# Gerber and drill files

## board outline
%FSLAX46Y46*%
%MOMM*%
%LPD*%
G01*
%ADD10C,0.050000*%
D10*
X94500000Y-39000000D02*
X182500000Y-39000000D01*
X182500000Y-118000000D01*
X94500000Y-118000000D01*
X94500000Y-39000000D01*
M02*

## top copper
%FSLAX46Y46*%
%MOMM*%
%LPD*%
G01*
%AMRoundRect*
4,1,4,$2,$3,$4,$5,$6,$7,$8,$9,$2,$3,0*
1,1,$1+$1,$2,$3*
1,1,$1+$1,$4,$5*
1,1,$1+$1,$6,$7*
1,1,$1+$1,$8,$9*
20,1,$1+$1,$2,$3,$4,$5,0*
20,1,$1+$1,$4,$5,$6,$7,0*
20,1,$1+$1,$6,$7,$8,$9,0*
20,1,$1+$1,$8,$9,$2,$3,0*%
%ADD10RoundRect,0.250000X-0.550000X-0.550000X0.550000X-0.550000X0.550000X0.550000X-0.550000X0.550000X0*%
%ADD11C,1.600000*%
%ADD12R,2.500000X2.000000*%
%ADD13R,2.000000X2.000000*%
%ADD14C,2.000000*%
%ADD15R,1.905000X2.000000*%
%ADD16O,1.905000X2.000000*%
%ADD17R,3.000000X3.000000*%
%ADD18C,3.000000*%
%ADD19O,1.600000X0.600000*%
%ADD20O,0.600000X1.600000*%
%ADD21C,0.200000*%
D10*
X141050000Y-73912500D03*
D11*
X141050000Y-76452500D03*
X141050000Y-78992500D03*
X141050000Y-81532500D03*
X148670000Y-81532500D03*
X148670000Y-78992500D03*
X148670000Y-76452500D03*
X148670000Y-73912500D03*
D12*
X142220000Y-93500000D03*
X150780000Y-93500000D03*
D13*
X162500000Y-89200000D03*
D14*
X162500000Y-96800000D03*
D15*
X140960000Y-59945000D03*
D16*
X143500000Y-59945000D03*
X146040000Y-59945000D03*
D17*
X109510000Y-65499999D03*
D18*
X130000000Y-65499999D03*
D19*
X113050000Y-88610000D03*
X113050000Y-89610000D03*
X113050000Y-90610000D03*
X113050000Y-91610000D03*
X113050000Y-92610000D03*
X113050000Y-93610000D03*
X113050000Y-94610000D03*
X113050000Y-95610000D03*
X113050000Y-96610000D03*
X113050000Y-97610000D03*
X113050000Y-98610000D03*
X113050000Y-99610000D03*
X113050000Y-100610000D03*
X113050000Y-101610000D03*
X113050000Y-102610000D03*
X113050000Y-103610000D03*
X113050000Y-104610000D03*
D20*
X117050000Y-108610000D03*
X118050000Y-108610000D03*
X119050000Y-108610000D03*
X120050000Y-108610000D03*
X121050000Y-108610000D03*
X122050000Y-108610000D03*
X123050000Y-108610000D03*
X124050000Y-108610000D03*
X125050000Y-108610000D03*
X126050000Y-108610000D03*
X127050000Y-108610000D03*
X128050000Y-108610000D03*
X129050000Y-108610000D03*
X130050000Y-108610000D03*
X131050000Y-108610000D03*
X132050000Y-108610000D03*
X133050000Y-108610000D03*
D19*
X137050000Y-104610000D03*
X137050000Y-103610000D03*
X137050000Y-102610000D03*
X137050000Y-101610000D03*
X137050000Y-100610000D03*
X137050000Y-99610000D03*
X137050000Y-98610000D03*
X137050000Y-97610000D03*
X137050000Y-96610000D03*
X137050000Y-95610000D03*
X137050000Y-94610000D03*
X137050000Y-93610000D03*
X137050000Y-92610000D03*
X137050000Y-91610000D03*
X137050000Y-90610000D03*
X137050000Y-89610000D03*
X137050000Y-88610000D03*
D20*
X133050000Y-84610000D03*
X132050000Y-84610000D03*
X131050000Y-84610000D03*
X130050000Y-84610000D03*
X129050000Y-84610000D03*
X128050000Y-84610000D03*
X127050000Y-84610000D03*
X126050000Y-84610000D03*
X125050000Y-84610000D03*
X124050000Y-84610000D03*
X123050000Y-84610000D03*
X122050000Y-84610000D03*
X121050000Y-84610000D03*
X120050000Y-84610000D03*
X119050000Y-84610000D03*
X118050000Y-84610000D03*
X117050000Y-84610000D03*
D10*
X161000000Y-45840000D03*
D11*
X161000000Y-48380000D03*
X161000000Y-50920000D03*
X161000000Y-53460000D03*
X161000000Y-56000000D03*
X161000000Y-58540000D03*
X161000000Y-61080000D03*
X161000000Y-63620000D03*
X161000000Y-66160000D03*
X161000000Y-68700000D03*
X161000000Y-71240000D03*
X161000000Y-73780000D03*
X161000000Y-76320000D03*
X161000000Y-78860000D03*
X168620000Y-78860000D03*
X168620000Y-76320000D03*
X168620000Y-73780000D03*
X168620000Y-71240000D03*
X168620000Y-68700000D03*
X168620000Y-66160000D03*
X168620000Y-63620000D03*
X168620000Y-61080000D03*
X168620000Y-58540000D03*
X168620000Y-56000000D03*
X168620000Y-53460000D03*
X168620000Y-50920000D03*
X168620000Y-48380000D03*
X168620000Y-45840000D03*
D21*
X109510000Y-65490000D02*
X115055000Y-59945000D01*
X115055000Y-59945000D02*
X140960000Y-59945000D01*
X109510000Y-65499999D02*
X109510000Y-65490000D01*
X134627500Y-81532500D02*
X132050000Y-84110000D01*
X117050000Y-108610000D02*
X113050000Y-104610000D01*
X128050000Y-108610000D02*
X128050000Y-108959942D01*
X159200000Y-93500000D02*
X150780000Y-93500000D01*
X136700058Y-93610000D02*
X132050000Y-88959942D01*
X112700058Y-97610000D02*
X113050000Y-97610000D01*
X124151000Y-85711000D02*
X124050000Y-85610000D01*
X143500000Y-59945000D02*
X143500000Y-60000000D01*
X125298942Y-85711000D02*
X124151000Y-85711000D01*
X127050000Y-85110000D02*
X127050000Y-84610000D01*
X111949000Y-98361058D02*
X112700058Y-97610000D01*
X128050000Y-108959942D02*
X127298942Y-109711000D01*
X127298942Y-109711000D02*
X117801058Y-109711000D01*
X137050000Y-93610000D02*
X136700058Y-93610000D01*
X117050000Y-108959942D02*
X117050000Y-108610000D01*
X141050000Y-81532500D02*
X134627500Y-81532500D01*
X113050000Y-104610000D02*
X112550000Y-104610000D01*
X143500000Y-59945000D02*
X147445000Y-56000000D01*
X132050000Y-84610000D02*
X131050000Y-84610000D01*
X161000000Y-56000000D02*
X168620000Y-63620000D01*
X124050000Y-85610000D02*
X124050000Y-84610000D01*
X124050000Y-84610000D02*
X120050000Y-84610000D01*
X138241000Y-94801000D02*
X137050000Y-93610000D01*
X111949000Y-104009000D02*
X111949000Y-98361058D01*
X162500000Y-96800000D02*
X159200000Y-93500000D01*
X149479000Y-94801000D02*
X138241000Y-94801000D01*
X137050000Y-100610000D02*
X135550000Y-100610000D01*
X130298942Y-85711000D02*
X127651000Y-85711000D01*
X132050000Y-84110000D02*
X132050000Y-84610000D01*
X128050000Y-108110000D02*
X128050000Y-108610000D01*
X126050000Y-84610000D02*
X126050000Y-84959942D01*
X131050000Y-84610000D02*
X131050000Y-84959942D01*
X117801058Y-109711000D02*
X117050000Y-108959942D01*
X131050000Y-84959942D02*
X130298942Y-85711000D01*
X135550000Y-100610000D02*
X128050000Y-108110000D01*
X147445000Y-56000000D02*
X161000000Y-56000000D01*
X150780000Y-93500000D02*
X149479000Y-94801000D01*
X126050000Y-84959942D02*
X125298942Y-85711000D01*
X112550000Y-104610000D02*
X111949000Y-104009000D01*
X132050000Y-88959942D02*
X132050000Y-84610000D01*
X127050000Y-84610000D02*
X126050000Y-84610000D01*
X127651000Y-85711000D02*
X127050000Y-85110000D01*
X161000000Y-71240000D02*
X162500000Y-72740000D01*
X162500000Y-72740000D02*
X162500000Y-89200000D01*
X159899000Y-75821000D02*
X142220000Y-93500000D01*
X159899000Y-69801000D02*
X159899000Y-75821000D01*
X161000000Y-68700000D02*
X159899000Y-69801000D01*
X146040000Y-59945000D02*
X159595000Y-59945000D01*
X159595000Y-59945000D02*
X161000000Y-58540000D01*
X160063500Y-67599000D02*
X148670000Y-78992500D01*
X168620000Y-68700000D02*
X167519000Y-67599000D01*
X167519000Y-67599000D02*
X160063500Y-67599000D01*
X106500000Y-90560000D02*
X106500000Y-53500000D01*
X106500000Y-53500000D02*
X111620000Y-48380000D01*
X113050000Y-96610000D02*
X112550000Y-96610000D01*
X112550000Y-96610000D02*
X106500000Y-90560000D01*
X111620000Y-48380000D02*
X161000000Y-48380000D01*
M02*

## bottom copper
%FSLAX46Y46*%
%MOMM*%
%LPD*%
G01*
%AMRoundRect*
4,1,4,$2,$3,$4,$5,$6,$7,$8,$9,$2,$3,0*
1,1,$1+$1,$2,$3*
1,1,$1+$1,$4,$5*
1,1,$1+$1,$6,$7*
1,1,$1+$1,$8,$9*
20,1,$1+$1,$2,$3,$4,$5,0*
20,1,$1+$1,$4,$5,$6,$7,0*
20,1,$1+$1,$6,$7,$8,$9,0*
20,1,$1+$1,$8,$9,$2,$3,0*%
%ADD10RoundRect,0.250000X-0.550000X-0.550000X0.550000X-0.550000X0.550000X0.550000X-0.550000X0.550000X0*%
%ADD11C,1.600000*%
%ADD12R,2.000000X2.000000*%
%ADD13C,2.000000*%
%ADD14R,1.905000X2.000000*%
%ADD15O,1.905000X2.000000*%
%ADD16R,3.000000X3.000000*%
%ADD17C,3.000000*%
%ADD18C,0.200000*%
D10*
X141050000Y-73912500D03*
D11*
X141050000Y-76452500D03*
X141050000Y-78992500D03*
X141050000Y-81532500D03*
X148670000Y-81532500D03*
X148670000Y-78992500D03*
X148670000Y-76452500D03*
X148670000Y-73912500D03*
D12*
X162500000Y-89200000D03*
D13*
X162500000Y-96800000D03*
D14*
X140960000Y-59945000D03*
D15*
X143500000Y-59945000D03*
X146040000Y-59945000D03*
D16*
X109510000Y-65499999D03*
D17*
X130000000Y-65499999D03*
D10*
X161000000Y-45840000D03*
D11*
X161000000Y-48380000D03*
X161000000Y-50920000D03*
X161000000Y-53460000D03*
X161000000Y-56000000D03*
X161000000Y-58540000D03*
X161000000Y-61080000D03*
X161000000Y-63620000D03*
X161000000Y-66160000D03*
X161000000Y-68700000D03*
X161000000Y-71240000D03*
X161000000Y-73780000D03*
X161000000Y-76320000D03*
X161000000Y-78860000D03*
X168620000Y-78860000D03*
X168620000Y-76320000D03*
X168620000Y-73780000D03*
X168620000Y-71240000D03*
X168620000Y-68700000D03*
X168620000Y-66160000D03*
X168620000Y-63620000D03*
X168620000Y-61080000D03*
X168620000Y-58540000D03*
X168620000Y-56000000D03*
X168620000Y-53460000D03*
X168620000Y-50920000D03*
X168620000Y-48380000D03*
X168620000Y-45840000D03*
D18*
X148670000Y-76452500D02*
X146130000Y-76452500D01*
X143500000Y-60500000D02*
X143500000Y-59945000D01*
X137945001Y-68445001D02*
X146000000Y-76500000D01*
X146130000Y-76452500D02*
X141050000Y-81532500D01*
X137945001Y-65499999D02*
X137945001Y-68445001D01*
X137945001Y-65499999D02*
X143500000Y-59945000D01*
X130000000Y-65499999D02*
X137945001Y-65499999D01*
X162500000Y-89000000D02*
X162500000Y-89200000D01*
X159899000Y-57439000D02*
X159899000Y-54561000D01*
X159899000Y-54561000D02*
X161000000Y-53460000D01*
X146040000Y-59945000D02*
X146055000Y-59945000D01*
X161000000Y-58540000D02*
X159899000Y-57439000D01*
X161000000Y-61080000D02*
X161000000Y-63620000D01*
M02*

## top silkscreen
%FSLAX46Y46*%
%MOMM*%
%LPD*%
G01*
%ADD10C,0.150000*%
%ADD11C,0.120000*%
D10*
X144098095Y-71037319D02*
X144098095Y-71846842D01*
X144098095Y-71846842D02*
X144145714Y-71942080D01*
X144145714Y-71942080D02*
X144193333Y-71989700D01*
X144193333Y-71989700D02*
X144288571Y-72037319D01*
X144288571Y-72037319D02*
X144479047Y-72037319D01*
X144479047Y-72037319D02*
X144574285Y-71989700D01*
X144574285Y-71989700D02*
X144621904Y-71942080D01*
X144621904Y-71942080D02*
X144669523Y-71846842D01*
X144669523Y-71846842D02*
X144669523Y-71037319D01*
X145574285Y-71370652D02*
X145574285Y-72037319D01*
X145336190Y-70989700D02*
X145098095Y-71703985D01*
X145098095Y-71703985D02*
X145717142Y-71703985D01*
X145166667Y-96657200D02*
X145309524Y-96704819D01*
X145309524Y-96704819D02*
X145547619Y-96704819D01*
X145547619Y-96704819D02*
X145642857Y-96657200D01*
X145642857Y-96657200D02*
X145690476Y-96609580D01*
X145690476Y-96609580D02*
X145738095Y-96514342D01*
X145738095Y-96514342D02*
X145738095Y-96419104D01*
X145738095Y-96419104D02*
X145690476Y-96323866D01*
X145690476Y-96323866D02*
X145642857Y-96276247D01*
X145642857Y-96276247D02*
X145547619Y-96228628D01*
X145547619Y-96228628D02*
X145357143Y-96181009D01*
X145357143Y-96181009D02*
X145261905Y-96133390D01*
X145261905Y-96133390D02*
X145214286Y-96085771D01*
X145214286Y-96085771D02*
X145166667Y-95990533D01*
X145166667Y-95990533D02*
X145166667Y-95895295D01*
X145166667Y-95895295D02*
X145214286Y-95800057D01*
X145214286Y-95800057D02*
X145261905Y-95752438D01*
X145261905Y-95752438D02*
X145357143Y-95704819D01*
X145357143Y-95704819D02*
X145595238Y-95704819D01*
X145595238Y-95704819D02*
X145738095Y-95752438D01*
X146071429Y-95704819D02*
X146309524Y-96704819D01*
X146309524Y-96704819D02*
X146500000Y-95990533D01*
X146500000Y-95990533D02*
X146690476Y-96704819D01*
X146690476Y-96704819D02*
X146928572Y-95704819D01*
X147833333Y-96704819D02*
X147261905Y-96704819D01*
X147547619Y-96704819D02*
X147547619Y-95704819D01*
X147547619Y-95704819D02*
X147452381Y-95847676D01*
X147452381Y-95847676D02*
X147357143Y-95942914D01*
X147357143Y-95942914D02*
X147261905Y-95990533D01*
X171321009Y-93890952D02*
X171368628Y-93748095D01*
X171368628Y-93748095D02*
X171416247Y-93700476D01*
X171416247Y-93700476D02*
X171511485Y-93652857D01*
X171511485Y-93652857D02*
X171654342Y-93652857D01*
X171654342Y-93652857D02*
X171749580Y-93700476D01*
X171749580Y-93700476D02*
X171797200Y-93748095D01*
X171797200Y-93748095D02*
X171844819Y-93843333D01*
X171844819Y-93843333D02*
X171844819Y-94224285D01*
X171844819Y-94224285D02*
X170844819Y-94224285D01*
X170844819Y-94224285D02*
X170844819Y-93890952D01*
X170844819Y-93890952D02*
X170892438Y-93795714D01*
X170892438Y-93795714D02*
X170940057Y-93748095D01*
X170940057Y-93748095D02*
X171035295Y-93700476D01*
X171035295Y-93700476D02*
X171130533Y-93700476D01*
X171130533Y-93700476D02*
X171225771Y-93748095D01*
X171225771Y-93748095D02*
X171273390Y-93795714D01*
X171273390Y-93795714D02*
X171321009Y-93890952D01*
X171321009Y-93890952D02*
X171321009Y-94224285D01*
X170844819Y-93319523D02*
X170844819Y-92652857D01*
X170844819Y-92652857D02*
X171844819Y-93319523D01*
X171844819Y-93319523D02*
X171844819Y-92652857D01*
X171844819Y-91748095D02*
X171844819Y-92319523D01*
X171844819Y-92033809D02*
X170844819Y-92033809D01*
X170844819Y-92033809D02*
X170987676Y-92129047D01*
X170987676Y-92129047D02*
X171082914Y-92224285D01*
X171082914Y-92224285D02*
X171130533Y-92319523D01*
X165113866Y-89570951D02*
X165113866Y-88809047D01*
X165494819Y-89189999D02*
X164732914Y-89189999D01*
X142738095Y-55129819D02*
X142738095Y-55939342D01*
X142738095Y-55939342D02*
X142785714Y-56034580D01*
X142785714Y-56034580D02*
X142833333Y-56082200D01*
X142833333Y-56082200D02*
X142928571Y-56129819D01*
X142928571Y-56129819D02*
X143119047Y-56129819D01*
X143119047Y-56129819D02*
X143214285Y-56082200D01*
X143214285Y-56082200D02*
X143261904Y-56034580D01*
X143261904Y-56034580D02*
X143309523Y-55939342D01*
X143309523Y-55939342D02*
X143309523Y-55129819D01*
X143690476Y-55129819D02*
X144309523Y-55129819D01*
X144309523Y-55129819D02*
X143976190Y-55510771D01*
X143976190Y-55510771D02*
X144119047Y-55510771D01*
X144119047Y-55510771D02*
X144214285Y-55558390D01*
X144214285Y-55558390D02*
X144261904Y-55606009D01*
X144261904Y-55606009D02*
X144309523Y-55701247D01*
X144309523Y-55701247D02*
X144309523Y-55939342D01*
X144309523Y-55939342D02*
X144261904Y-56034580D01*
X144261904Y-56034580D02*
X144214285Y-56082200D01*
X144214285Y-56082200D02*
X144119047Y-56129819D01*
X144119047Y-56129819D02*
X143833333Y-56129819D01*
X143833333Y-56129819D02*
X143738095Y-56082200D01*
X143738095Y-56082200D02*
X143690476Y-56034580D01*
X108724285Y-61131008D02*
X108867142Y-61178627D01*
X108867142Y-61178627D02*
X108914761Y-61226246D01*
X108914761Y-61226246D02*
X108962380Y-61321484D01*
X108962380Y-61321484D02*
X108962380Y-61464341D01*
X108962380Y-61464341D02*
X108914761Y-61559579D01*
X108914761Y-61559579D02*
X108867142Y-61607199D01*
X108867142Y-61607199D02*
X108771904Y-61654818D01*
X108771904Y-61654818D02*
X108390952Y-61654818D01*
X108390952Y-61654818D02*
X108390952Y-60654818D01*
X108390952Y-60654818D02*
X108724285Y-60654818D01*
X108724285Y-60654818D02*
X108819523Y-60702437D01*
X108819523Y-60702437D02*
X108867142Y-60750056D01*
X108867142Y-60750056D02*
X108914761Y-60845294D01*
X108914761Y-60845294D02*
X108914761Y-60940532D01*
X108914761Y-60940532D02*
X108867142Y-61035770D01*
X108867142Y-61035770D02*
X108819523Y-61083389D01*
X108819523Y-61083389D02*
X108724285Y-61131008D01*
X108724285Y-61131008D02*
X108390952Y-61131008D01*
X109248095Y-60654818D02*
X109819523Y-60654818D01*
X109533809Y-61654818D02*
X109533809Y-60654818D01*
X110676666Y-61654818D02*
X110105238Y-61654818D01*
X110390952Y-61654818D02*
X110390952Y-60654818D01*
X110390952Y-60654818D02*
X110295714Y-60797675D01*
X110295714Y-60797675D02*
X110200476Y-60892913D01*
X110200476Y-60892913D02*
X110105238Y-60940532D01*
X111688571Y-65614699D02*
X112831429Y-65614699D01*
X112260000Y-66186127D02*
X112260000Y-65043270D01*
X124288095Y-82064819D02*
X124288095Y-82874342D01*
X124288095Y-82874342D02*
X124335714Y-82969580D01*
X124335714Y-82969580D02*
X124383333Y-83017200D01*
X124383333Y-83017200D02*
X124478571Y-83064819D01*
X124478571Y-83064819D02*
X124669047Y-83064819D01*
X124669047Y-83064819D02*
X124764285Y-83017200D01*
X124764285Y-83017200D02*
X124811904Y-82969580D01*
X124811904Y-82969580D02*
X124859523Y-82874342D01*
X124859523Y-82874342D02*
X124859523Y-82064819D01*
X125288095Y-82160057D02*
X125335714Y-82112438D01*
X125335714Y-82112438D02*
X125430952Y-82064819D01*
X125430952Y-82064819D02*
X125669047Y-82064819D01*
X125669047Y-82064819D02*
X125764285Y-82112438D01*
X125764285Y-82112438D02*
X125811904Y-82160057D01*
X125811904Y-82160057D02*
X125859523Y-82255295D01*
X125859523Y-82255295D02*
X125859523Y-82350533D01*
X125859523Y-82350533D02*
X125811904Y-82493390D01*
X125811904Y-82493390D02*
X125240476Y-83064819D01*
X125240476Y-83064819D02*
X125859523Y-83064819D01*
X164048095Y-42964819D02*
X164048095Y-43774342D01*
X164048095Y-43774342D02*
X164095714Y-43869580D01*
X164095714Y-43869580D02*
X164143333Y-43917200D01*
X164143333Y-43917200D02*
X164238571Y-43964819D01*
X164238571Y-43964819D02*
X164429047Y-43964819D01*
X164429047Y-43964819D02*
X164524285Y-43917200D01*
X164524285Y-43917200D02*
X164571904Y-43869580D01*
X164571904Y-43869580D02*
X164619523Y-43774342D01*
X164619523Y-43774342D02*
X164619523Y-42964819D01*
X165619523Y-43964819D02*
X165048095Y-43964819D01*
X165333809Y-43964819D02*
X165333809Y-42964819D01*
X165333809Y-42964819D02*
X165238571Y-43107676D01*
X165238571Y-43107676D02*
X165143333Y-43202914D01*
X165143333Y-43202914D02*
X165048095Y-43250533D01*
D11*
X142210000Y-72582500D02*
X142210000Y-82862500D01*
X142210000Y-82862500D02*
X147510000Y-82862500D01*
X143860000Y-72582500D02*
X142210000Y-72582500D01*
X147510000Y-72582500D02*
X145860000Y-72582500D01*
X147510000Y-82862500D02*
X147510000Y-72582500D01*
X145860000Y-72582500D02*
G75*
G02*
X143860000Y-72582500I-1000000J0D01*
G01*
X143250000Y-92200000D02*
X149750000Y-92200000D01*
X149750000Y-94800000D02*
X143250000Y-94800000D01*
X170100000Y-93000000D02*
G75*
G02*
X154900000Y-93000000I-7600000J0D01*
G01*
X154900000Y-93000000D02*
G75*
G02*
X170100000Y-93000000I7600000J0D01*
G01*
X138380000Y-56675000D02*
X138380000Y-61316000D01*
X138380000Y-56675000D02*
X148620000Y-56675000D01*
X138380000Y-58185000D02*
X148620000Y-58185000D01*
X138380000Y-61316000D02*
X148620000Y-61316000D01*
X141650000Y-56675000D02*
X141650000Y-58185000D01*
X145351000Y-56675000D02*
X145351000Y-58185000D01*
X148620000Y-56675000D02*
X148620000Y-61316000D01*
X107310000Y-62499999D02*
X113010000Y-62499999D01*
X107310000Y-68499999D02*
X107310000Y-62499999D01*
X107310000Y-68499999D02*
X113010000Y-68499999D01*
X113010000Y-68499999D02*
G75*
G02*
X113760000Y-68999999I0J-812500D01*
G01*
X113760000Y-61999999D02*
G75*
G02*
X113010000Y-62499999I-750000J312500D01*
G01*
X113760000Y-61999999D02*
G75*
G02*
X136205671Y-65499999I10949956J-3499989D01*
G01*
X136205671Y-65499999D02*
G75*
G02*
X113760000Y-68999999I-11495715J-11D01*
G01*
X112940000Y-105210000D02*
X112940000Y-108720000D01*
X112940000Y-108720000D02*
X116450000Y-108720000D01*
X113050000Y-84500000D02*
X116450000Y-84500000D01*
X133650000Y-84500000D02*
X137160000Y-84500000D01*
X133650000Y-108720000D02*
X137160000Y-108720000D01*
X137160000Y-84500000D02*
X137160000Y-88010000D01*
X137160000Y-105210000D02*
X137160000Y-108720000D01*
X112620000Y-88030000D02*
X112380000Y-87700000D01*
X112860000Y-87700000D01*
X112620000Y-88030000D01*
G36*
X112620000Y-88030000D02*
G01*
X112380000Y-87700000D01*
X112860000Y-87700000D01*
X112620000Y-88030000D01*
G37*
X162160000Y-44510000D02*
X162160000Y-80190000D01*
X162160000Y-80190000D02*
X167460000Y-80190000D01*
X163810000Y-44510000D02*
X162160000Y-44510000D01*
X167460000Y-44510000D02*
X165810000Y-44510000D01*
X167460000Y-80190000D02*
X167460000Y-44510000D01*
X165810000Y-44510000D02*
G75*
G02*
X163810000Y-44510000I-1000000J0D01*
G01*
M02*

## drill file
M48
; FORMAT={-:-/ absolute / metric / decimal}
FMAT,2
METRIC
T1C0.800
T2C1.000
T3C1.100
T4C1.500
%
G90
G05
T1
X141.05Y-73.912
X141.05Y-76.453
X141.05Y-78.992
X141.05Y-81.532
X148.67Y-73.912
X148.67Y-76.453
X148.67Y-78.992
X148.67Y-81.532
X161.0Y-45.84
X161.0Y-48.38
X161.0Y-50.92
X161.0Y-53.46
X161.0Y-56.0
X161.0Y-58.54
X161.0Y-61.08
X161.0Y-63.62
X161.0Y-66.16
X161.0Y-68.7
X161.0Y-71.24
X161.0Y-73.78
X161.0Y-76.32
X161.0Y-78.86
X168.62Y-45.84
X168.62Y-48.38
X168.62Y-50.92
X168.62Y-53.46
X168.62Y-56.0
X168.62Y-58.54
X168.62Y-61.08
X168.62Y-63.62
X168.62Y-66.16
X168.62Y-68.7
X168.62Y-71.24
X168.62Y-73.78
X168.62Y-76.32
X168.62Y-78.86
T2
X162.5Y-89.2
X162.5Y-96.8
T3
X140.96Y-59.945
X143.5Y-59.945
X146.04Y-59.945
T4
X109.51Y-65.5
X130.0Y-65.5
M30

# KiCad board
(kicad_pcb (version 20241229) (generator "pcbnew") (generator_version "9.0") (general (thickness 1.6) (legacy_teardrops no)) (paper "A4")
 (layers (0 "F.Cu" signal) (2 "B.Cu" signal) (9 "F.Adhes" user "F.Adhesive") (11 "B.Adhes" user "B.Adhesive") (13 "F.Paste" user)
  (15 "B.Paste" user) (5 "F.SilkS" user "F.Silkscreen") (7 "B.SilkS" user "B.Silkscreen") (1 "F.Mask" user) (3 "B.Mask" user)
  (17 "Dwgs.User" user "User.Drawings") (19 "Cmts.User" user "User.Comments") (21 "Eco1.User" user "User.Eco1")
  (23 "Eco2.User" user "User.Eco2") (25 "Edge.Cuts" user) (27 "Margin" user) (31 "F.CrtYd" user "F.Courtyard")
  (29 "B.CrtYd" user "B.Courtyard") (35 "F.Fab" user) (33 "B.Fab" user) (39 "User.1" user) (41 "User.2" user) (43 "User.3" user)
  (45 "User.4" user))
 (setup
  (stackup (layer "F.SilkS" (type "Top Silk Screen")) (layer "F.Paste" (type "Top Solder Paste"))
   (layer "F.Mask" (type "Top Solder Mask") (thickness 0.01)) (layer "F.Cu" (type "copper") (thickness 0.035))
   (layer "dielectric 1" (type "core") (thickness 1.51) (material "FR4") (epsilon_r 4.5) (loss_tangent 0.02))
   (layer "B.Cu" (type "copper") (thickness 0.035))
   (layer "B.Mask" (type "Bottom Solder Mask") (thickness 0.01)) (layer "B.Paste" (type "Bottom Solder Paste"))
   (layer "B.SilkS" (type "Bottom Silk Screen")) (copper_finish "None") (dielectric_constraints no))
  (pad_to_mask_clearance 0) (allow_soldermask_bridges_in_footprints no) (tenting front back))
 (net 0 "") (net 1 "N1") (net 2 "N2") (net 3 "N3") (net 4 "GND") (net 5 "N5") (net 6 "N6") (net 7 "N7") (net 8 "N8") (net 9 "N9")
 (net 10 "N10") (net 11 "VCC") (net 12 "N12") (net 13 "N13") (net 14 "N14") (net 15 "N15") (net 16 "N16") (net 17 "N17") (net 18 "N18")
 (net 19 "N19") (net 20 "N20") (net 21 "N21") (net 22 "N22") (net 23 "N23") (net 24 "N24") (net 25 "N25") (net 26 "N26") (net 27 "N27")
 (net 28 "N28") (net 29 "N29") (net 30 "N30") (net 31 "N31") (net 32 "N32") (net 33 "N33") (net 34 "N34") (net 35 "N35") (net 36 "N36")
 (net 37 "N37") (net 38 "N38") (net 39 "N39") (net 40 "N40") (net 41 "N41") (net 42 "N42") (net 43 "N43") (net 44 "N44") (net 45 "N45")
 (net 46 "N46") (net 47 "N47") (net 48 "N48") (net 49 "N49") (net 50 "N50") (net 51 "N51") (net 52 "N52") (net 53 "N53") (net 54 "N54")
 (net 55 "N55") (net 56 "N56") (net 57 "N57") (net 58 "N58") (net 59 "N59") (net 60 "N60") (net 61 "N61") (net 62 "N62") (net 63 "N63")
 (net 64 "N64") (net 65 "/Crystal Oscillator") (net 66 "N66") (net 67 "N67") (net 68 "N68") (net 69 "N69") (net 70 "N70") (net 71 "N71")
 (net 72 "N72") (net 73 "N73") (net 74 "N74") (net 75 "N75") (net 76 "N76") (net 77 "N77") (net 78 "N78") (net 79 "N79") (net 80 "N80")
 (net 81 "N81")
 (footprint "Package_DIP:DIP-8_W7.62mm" (layer "F.Cu") (at 141.05 73.9125)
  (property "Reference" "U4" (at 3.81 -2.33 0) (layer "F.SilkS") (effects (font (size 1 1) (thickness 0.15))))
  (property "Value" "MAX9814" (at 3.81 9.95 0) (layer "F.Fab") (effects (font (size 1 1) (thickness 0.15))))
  (fp_line (start 1.16 -1.33) (end 1.16 8.95) (stroke (width 0.12) (type solid)) (layer "F.SilkS"))
  (fp_line (start 1.16 8.95) (end 6.46 8.95) (stroke (width 0.12) (type solid)) (layer "F.SilkS"))
  (fp_line (start 2.81 -1.33) (end 1.16 -1.33) (stroke (width 0.12) (type solid)) (layer "F.SilkS"))
  (fp_line (start 6.46 -1.33) (end 4.81 -1.33) (stroke (width 0.12) (type solid)) (layer "F.SilkS"))
  (fp_line (start 6.46 8.95) (end 6.46 -1.33) (stroke (width 0.12) (type solid)) (layer "F.SilkS"))
  (fp_arc (start 4.81 -1.33) (mid 3.81 -0.33) (end 2.81 -1.33) (stroke (width 0.12) (type solid)) (layer "F.SilkS"))
  (pad "1" thru_hole roundrect (at 0 0) (size 1.6 1.6) (drill 0.8) (layers "*.Cu" "*.Mask") (remove_unused_layers no)
   (roundrect_rratio 0.15625) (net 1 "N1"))
  (pad "2" thru_hole circle (at 0 2.54) (size 1.6 1.6) (drill 0.8) (layers "*.Cu" "*.Mask") (remove_unused_layers no) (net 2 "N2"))
  (pad "3" thru_hole circle (at 0 5.08) (size 1.6 1.6) (drill 0.8) (layers "*.Cu" "*.Mask") (remove_unused_layers no) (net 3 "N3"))
  (pad "4" thru_hole circle (at 0 7.62) (size 1.6 1.6) (drill 0.8) (layers "*.Cu" "*.Mask") (remove_unused_layers no) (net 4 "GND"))
  (pad "5" thru_hole circle (at 7.62 7.62) (size 1.6 1.6) (drill 0.8) (layers "*.Cu" "*.Mask") (remove_unused_layers no) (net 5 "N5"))
  (pad "6" thru_hole circle (at 7.62 5.08) (size 1.6 1.6) (drill 0.8) (layers "*.Cu" "*.Mask") (remove_unused_layers no) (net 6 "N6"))
  (pad "7" thru_hole circle (at 7.62 2.54) (size 1.6 1.6) (drill 0.8) (layers "*.Cu" "*.Mask") (remove_unused_layers no) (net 4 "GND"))
  (pad "8" thru_hole circle (at 7.62 0) (size 1.6 1.6) (drill 0.8) (layers "*.Cu" "*.Mask") (remove_unused_layers no) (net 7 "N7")))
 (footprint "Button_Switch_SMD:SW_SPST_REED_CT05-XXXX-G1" (layer "F.Cu") (at 146.5 93.5)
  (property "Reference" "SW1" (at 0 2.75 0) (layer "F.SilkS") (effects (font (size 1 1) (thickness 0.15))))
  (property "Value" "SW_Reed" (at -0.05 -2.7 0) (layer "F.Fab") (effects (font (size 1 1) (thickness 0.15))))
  (fp_line (start -3.25 -1.3) (end 3.25 -1.3) (stroke (width 0.12) (type solid)) (layer "F.SilkS"))
  (fp_line (start 3.25 1.3) (end -3.25 1.3) (stroke (width 0.12) (type solid)) (layer "F.SilkS"))
  (pad "1" smd rect (at -4.28 0) (size 2.5 2) (layers "F.Cu" "F.Mask" "F.Paste") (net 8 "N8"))
  (pad "2" smd rect (at 4.28 0) (size 2.5 2) (layers "F.Cu" "F.Mask" "F.Paste") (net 4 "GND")))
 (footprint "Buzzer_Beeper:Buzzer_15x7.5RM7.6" (layer "F.Cu") (at 162.5 89.2 -90)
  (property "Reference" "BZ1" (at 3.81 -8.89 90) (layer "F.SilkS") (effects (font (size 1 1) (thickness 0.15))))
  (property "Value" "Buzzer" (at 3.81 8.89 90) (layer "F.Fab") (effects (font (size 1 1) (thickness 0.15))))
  (fp_circle (center 3.8 0) (end 11.4 0) (stroke (width 0.12) (type solid)) (fill no) (layer "F.SilkS"))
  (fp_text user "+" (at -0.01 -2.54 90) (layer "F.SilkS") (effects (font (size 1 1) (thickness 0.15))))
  (pad "1" thru_hole rect (at 0 0 270) (size 2 2) (drill 1) (layers "*.Cu" "*.Mask") (remove_unused_layers no) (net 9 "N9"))
  (pad "2" thru_hole circle (at 7.6 0 270) (size 2 2) (drill 1) (layers "*.Cu" "*.Mask") (remove_unused_layers no) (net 4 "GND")))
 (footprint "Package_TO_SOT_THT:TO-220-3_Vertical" (layer "F.Cu") (at 140.96 59.945)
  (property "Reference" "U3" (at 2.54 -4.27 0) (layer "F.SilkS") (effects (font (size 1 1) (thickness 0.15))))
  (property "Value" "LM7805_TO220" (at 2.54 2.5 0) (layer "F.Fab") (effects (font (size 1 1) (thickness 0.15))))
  (fp_line (start -2.58 -3.27) (end -2.58 1.371) (stroke (width 0.12) (type solid)) (layer "F.SilkS"))
  (fp_line (start -2.58 -3.27) (end 7.66 -3.27) (stroke (width 0.12) (type solid)) (layer "F.SilkS"))
  (fp_line (start -2.58 -1.76) (end 7.66 -1.76) (stroke (width 0.12) (type solid)) (layer "F.SilkS"))
  (fp_line (start -2.58 1.371) (end 7.66 1.371) (stroke (width 0.12) (type solid)) (layer "F.SilkS"))
  (fp_line (start 0.69 -3.27) (end 0.69 -1.76) (stroke (width 0.12) (type solid)) (layer "F.SilkS"))
  (fp_line (start 4.391 -3.27) (end 4.391 -1.76) (stroke (width 0.12) (type solid)) (layer "F.SilkS"))
  (fp_line (start 7.66 -3.27) (end 7.66 1.371) (stroke (width 0.12) (type solid)) (layer "F.SilkS"))
  (pad "1" thru_hole rect (at 0 0) (size 1.905 2) (drill 1.1) (layers "*.Cu" "*.Mask") (remove_unused_layers no) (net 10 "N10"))
  (pad "2" thru_hole oval (at 2.54 0) (size 1.905 2) (drill 1.1) (layers "*.Cu" "*.Mask") (remove_unused_layers no) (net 4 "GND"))
  (pad "3" thru_hole oval (at 5.08 0) (size 1.905 2) (drill 1.1) (layers "*.Cu" "*.Mask") (remove_unused_layers no) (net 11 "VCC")))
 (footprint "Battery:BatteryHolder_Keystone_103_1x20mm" (layer "F.Cu") (at 109.51 65.499999)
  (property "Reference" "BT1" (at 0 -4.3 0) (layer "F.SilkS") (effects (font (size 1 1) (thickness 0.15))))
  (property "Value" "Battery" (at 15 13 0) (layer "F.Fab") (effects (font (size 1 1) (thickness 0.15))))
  (fp_line (start -2.2 -3) (end 3.5 -3) (stroke (width 0.12) (type solid)) (layer "F.SilkS"))
  (fp_line (start -2.2 3) (end -2.2 -3) (stroke (width 0.12) (type solid)) (layer "F.SilkS"))
  (fp_line (start -2.2 3) (end 3.5 3) (stroke (width 0.12) (type solid)) (layer "F.SilkS"))
  (fp_arc (start 3.5 3) (mid 3.950694 3.136459) (end 4.25 3.5) (stroke (width 0.12) (type solid)) (layer "F.SilkS"))
  (fp_arc (start 4.25 -3.5) (mid 3.950694 -3.136459) (end 3.5 -3) (stroke (width 0.12) (type solid)) (layer "F.SilkS"))
  (fp_arc (start 4.25 -3.5) (mid 16.971103 -11.358466) (end 26.695671 0) (stroke (width 0.12) (type solid)) (layer "F.SilkS"))
  (fp_arc (start 26.695671 0) (mid 16.971103 11.358466) (end 4.25 3.5) (stroke (width 0.12) (type solid)) (layer "F.SilkS"))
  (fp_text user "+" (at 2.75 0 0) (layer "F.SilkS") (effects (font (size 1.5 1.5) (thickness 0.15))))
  (pad "1" thru_hole rect (at 0 0) (size 3 3) (drill 1.5) (layers "*.Cu" "*.Mask") (remove_unused_layers no) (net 10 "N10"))
  (pad "2" thru_hole circle (at 20.49 0) (size 3 3) (drill 1.5) (layers "*.Cu" "*.Mask") (remove_unused_layers no) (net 4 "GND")))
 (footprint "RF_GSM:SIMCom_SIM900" (layer "F.Cu") (at 125.05 96.61)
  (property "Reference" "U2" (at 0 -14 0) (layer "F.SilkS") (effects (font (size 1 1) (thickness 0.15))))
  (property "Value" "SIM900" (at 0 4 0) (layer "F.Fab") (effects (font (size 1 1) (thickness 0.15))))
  (fp_line (start -12.11 8.6) (end -12.11 12.11) (stroke (width 0.12) (type solid)) (layer "F.SilkS"))
  (fp_line (start -12.11 12.11) (end -8.6 12.11) (stroke (width 0.12) (type solid)) (layer "F.SilkS"))
  (fp_line (start -12 -12.11) (end -8.6 -12.11) (stroke (width 0.12) (type solid)) (layer "F.SilkS"))
  (fp_line (start 8.6 -12.11) (end 12.11 -12.11) (stroke (width 0.12) (type solid)) (layer "F.SilkS"))
  (fp_line (start 8.6 12.11) (end 12.11 12.11) (stroke (width 0.12) (type solid)) (layer "F.SilkS"))
  (fp_line (start 12.11 -12.11) (end 12.11 -8.6) (stroke (width 0.12) (type solid)) (layer "F.SilkS"))
  (fp_line (start 12.11 8.6) (end 12.11 12.11) (stroke (width 0.12) (type solid)) (layer "F.SilkS"))
  (fp_poly
   (pts (xy -12.43 -8.58) (xy -12.67 -8.91) (xy -12.19 -8.91) (xy -12.43 -8.58)) (stroke (width 0.12) (type solid)) (fill yes)
   (layer "F.SilkS"))
  (pad "1" smd oval (at -12 -8) (size 1.6 0.6) (layers "F.Cu" "F.Mask" "F.Paste") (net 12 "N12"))
  (pad "2" smd oval (at -12 -7) (size 1.6 0.6) (layers "F.Cu" "F.Mask" "F.Paste") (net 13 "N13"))
  (pad "3" smd oval (at -12 -6) (size 1.6 0.6) (layers "F.Cu" "F.Mask" "F.Paste") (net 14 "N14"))
  (pad "4" smd oval (at -12 -5) (size 1.6 0.6) (layers "F.Cu" "F.Mask" "F.Paste") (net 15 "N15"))
  (pad "5" smd oval (at -12 -4) (size 1.6 0.6) (layers "F.Cu" "F.Mask" "F.Paste") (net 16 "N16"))
  (pad "6" smd oval (at -12 -3) (size 1.6 0.6) (layers "F.Cu" "F.Mask" "F.Paste") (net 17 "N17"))
  (pad "7" smd oval (at -12 -2) (size 1.6 0.6) (layers "F.Cu" "F.Mask" "F.Paste") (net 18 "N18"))
  (pad "8" smd oval (at -12 -1) (size 1.6 0.6) (layers "F.Cu" "F.Mask" "F.Paste") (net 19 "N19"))
  (pad "9" smd oval (at -12 0) (size 1.6 0.6) (layers "F.Cu" "F.Mask" "F.Paste") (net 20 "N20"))
  (pad "10" smd oval (at -12 1) (size 1.6 0.6) (layers "F.Cu" "F.Mask" "F.Paste") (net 4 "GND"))
  (pad "11" smd oval (at -12 2) (size 1.6 0.6) (layers "F.Cu" "F.Mask" "F.Paste") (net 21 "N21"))
  (pad "12" smd oval (at -12 3) (size 1.6 0.6) (layers "F.Cu" "F.Mask" "F.Paste") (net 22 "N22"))
  (pad "13" smd oval (at -12 4) (size 1.6 0.6) (layers "F.Cu" "F.Mask" "F.Paste") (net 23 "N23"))
  (pad "14" smd oval (at -12 5) (size 1.6 0.6) (layers "F.Cu" "F.Mask" "F.Paste") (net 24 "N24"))
  (pad "15" smd oval (at -12 6) (size 1.6 0.6) (layers "F.Cu" "F.Mask" "F.Paste") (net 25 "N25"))
  (pad "16" smd oval (at -12 7) (size 1.6 0.6) (layers "F.Cu" "F.Mask" "F.Paste") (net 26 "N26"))
  (pad "17" smd oval (at -12 8) (size 1.6 0.6) (layers "F.Cu" "F.Mask" "F.Paste") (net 4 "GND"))
  (pad "18" smd oval (at -8 12) (size 0.6 1.6) (layers "F.Cu" "F.Mask" "F.Paste") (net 4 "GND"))
  (pad "19" smd oval (at -7 12) (size 0.6 1.6) (layers "F.Cu" "F.Mask" "F.Paste") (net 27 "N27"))
  (pad "20" smd oval (at -6 12) (size 0.6 1.6) (layers "F.Cu" "F.Mask" "F.Paste") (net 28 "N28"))
  (pad "21" smd oval (at -5 12) (size 0.6 1.6) (layers "F.Cu" "F.Mask" "F.Paste") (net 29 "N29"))
  (pad "22" smd oval (at -4 12) (size 0.6 1.6) (layers "F.Cu" "F.Mask" "F.Paste") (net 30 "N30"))
  (pad "23" smd oval (at -3 12) (size 0.6 1.6) (layers "F.Cu" "F.Mask" "F.Paste") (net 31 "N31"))
  (pad "24" smd oval (at -2 12) (size 0.6 1.6) (layers "F.Cu" "F.Mask" "F.Paste") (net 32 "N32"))
  (pad "25" smd oval (at -1 12) (size 0.6 1.6) (layers "F.Cu" "F.Mask" "F.Paste") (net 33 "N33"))
  (pad "26" smd oval (at 0 12) (size 0.6 1.6) (layers "F.Cu" "F.Mask" "F.Paste") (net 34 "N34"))
  (pad "27" smd oval (at 1 12) (size 0.6 1.6) (layers "F.Cu" "F.Mask" "F.Paste") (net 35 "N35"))
  (pad "28" smd oval (at 2 12) (size 0.6 1.6) (layers "F.Cu" "F.Mask" "F.Paste") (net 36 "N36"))
  (pad "29" smd oval (at 3 12) (size 0.6 1.6) (layers "F.Cu" "F.Mask" "F.Paste") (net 4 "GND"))
  (pad "30" smd oval (at 4 12) (size 0.6 1.6) (layers "F.Cu" "F.Mask" "F.Paste") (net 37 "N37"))
  (pad "31" smd oval (at 5 12) (size 0.6 1.6) (layers "F.Cu" "F.Mask" "F.Paste") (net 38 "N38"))
  (pad "32" smd oval (at 6 12) (size 0.6 1.6) (layers "F.Cu" "F.Mask" "F.Paste") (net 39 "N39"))
  (pad "33" smd oval (at 7 12) (size 0.6 1.6) (layers "F.Cu" "F.Mask" "F.Paste") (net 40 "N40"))
  (pad "34" smd oval (at 8 12) (size 0.6 1.6) (layers "F.Cu" "F.Mask" "F.Paste") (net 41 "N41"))
  (pad "35" smd oval (at 12 8) (size 1.6 0.6) (layers "F.Cu" "F.Mask" "F.Paste") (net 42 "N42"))
  (pad "36" smd oval (at 12 7) (size 1.6 0.6) (layers "F.Cu" "F.Mask" "F.Paste") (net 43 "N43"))
  (pad "37" smd oval (at 12 6) (size 1.6 0.6) (layers "F.Cu" "F.Mask" "F.Paste") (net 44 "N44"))
  (pad "38" smd oval (at 12 5) (size 1.6 0.6) (layers "F.Cu" "F.Mask" "F.Paste") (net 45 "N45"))
  (pad "39" smd oval (at 12 4) (size 1.6 0.6) (layers "F.Cu" "F.Mask" "F.Paste") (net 4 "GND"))
  (pad "40" smd oval (at 12 3) (size 1.6 0.6) (layers "F.Cu" "F.Mask" "F.Paste") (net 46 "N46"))
  (pad "41" smd oval (at 12 2) (size 1.6 0.6) (layers "F.Cu" "F.Mask" "F.Paste") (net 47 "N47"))
  (pad "42" smd oval (at 12 1) (size 1.6 0.6) (layers "F.Cu" "F.Mask" "F.Paste") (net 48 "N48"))
  (pad "43" smd oval (at 12 0) (size 1.6 0.6) (layers "F.Cu" "F.Mask" "F.Paste") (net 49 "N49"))
  (pad "44" smd oval (at 12 -1) (size 1.6 0.6) (layers "F.Cu" "F.Mask" "F.Paste") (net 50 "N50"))
  (pad "45" smd oval (at 12 -2) (size 1.6 0.6) (layers "F.Cu" "F.Mask" "F.Paste") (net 4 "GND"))
  (pad "46" smd oval (at 12 -3) (size 1.6 0.6) (layers "F.Cu" "F.Mask" "F.Paste") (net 4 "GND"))
  (pad "47" smd oval (at 12 -4) (size 1.6 0.6) (layers "F.Cu" "F.Mask" "F.Paste") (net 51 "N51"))
  (pad "48" smd oval (at 12 -5) (size 1.6 0.6) (layers "F.Cu" "F.Mask" "F.Paste") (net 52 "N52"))
  (pad "49" smd oval (at 12 -6) (size 1.6 0.6) (layers "F.Cu" "F.Mask" "F.Paste") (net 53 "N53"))
  (pad "50" smd oval (at 12 -7) (size 1.6 0.6) (layers "F.Cu" "F.Mask" "F.Paste") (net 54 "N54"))
  (pad "51" smd oval (at 12 -8) (size 1.6 0.6) (layers "F.Cu" "F.Mask" "F.Paste") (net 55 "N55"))
  (pad "52" smd oval (at 8 -12) (size 0.6 1.6) (layers "F.Cu" "F.Mask" "F.Paste") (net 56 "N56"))
  (pad "53" smd oval (at 7 -12) (size 0.6 1.6) (layers "F.Cu" "F.Mask" "F.Paste") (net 4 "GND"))
  (pad "54" smd oval (at 6 -12) (size 0.6 1.6) (layers "F.Cu" "F.Mask" "F.Paste") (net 4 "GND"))
  (pad "55" smd oval (at 5 -12) (size 0.6 1.6) (layers "F.Cu" "F.Mask" "F.Paste") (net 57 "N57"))
  (pad "56" smd oval (at 4 -12) (size 0.6 1.6) (layers "F.Cu" "F.Mask" "F.Paste") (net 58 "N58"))
  (pad "57" smd oval (at 3 -12) (size 0.6 1.6) (layers "F.Cu" "F.Mask" "F.Paste") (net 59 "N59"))
  (pad "58" smd oval (at 2 -12) (size 0.6 1.6) (layers "F.Cu" "F.Mask" "F.Paste") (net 4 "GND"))
  (pad "59" smd oval (at 1 -12) (size 0.6 1.6) (layers "F.Cu" "F.Mask" "F.Paste") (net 4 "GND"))
  (pad "60" smd oval (at 0 -12) (size 0.6 1.6) (layers "F.Cu" "F.Mask" "F.Paste") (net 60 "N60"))
  (pad "61" smd oval (at -1 -12) (size 0.6 1.6) (layers "F.Cu" "F.Mask" "F.Paste") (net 4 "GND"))
  (pad "62" smd oval (at -2 -12) (size 0.6 1.6) (layers "F.Cu" "F.Mask" "F.Paste") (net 4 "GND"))
  (pad "63" smd oval (at -3 -12) (size 0.6 1.6) (layers "F.Cu" "F.Mask" "F.Paste") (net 4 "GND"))
  (pad "64" smd oval (at -4 -12) (size 0.6 1.6) (layers "F.Cu" "F.Mask" "F.Paste") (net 4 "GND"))
  (pad "65" smd oval (at -5 -12) (size 0.6 1.6) (layers "F.Cu" "F.Mask" "F.Paste") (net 4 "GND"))
  (pad "66" smd oval (at -6 -12) (size 0.6 1.6) (layers "F.Cu" "F.Mask" "F.Paste") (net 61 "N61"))
  (pad "67" smd oval (at -7 -12) (size 0.6 1.6) (layers "F.Cu" "F.Mask" "F.Paste") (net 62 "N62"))
  (pad "68" smd oval (at -8 -12) (size 0.6 1.6) (layers "F.Cu" "F.Mask" "F.Paste") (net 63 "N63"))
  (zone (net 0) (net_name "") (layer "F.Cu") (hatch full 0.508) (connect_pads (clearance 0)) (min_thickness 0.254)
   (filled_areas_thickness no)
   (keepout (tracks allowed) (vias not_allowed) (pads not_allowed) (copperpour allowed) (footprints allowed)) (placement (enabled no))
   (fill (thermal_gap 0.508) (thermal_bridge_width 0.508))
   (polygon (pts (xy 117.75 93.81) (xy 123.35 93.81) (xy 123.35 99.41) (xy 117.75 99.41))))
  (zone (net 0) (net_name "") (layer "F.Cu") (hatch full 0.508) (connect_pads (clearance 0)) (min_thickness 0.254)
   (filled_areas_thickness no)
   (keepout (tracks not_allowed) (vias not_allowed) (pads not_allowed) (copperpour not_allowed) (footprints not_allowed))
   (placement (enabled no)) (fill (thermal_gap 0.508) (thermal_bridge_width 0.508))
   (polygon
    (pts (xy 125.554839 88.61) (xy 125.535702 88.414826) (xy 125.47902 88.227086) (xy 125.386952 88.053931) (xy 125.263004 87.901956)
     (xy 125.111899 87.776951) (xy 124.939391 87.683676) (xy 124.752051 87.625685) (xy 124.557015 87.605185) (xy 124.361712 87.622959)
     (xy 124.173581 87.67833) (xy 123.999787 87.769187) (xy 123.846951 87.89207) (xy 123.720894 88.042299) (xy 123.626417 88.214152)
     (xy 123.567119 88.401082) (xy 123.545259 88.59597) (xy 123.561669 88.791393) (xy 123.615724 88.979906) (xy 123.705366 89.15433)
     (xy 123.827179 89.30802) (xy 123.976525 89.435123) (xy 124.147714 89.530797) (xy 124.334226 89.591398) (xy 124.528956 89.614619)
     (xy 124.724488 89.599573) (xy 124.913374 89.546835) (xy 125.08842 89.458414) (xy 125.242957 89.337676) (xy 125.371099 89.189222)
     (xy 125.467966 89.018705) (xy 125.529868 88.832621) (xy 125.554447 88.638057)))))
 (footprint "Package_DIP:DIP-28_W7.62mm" (layer "F.Cu") (at 161 45.84)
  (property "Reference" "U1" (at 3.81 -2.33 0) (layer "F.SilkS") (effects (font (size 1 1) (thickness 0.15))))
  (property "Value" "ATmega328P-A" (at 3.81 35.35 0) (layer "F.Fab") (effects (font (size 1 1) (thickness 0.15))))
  (fp_line (start 1.16 -1.33) (end 1.16 34.35) (stroke (width 0.12) (type solid)) (layer "F.SilkS"))
  (fp_line (start 1.16 34.35) (end 6.46 34.35) (stroke (width 0.12) (type solid)) (layer "F.SilkS"))
  (fp_line (start 2.81 -1.33) (end 1.16 -1.33) (stroke (width 0.12) (type solid)) (layer "F.SilkS"))
  (fp_line (start 6.46 -1.33) (end 4.81 -1.33) (stroke (width 0.12) (type solid)) (layer "F.SilkS"))
  (fp_line (start 6.46 34.35) (end 6.46 -1.33) (stroke (width 0.12) (type solid)) (layer "F.SilkS"))
  (fp_arc (start 4.81 -1.33) (mid 3.81 -0.33) (end 2.81 -1.33) (stroke (width 0.12) (type solid)) (layer "F.SilkS"))
  (pad "1" thru_hole roundrect (at 0 0) (size 1.6 1.6) (drill 0.8) (layers "*.Cu" "*.Mask") (remove_unused_layers no)
   (roundrect_rratio 0.15625) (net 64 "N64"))
  (pad "2" thru_hole circle (at 0 2.54) (size 1.6 1.6) (drill 0.8) (layers "*.Cu" "*.Mask") (remove_unused_layers no) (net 20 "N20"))
  (pad "3" thru_hole circle (at 0 5.08) (size 1.6 1.6) (drill 0.8) (layers "*.Cu" "*.Mask") (remove_unused_layers no) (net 4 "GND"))
  (pad "4" thru_hole circle (at 0 7.62) (size 1.6 1.6) (drill 0.8) (layers "*.Cu" "*.Mask") (remove_unused_layers no) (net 11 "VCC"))
  (pad "5" thru_hole circle (at 0 10.16) (size 1.6 1.6) (drill 0.8) (layers "*.Cu" "*.Mask") (remove_unused_layers no) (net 4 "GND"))
  (pad "6" thru_hole circle (at 0 12.7) (size 1.6 1.6) (drill 0.8) (layers "*.Cu" "*.Mask") (remove_unused_layers no) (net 11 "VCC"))
  (pad "7" thru_hole circle (at 0 15.24) (size 1.6 1.6) (drill 0.8) (layers "*.Cu" "*.Mask") (remove_unused_layers no)
   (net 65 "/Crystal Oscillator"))
  (pad "8" thru_hole circle (at 0 17.78) (size 1.6 1.6) (drill 0.8) (layers "*.Cu" "*.Mask") (remove_unused_layers no)
   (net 65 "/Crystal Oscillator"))
  (pad "9" thru_hole circle (at 0 20.32) (size 1.6 1.6) (drill 0.8) (layers "*.Cu" "*.Mask") (remove_unused_layers no) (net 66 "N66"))
  (pad "10" thru_hole circle (at 0 22.86) (size 1.6 1.6) (drill 0.8) (layers "*.Cu" "*.Mask") (remove_unused_layers no) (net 8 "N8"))
  (pad "11" thru_hole circle (at 0 25.4) (size 1.6 1.6) (drill 0.8) (layers "*.Cu" "*.Mask") (remove_unused_layers no) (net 9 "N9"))
  (pad "12" thru_hole circle (at 0 27.94) (size 1.6 1.6) (drill 0.8) (layers "*.Cu" "*.Mask") (remove_unused_layers no) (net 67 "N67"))
  (pad "13" thru_hole circle (at 0 30.48) (size 1.6 1.6) (drill 0.8) (layers "*.Cu" "*.Mask") (remove_unused_layers no) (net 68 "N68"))
  (pad "14" thru_hole circle (at 0 33.02) (size 1.6 1.6) (drill 0.8) (layers "*.Cu" "*.Mask") (remove_unused_layers no) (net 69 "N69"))
  (pad "15" thru_hole circle (at 7.62 33.02) (size 1.6 1.6) (drill 0.8) (layers "*.Cu" "*.Mask") (remove_unused_layers no) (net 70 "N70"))
  (pad "16" thru_hole circle (at 7.62 30.48) (size 1.6 1.6) (drill 0.8) (layers "*.Cu" "*.Mask") (remove_unused_layers no) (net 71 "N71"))
  (pad "17" thru_hole circle (at 7.62 27.94) (size 1.6 1.6) (drill 0.8) (layers "*.Cu" "*.Mask") (remove_unused_layers no) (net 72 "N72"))
  (pad "18" thru_hole circle (at 7.62 25.4) (size 1.6 1.6) (drill 0.8) (layers "*.Cu" "*.Mask") (remove_unused_layers no) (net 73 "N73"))
  (pad "19" thru_hole circle (at 7.62 22.86) (size 1.6 1.6) (drill 0.8) (layers "*.Cu" "*.Mask") (remove_unused_layers no) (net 6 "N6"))
  (pad "20" thru_hole circle (at 7.62 20.32) (size 1.6 1.6) (drill 0.8) (layers "*.Cu" "*.Mask") (remove_unused_layers no) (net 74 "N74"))
  (pad "21" thru_hole circle (at 7.62 17.78) (size 1.6 1.6) (drill 0.8) (layers "*.Cu" "*.Mask") (remove_unused_layers no) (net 4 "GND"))
  (pad "22" thru_hole circle (at 7.62 15.24) (size 1.6 1.6) (drill 0.8) (layers "*.Cu" "*.Mask") (remove_unused_layers no) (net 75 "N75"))
  (pad "23" thru_hole circle (at 7.62 12.7) (size 1.6 1.6) (drill 0.8) (layers "*.Cu" "*.Mask") (remove_unused_layers no) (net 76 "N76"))
  (pad "24" thru_hole circle (at 7.62 10.16) (size 1.6 1.6) (drill 0.8) (layers "*.Cu" "*.Mask") (remove_unused_layers no) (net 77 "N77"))
  (pad "25" thru_hole circle (at 7.62 7.62) (size 1.6 1.6) (drill 0.8) (layers "*.Cu" "*.Mask") (remove_unused_layers no) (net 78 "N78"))
  (pad "26" thru_hole circle (at 7.62 5.08) (size 1.6 1.6) (drill 0.8) (layers "*.Cu" "*.Mask") (remove_unused_layers no) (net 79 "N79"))
  (pad "27" thru_hole circle (at 7.62 2.54) (size 1.6 1.6) (drill 0.8) (layers "*.Cu" "*.Mask") (remove_unused_layers no) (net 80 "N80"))
  (pad "28" thru_hole circle (at 7.62 0) (size 1.6 1.6) (drill 0.8) (layers "*.Cu" "*.Mask") (remove_unused_layers no) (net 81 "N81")))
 (gr_rect (start 94.5 39) (end 182.5 118) (stroke (width 0.05) (type default)) (fill no) (layer "Edge.Cuts"))
 (segment (start 109.51 65.49) (end 115.055 59.945) (width 0.2) (layer "F.Cu") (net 10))
 (segment (start 115.055 59.945) (end 140.96 59.945) (width 0.2) (layer "F.Cu") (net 10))
 (segment (start 109.51 65.499999) (end 109.51 65.49) (width 0.2) (layer "F.Cu") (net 10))
 (segment (start 134.6275 81.5325) (end 132.05 84.11) (width 0.2) (layer "F.Cu") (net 4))
 (segment (start 117.05 108.61) (end 113.05 104.61) (width 0.2) (layer "F.Cu") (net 4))
 (segment (start 128.05 108.61) (end 128.05 108.959942) (width 0.2) (layer "F.Cu") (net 4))
 (segment (start 159.2 93.5) (end 150.78 93.5) (width 0.2) (layer "F.Cu") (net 4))
 (segment (start 136.700058 93.61) (end 132.05 88.959942) (width 0.2) (layer "F.Cu") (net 4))
 (segment (start 112.700058 97.61) (end 113.05 97.61) (width 0.2) (layer "F.Cu") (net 4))
 (segment (start 124.151 85.711) (end 124.05 85.61) (width 0.2) (layer "F.Cu") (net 4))
 (segment (start 143.5 59.945) (end 143.5 60) (width 0.2) (layer "F.Cu") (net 4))
 (segment (start 125.298942 85.711) (end 124.151 85.711) (width 0.2) (layer "F.Cu") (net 4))
 (segment (start 127.05 85.11) (end 127.05 84.61) (width 0.2) (layer "F.Cu") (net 4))
 (segment (start 111.949 98.361058) (end 112.700058 97.61) (width 0.2) (layer "F.Cu") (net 4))
 (segment (start 128.05 108.959942) (end 127.298942 109.711) (width 0.2) (layer "F.Cu") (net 4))
 (segment (start 127.298942 109.711) (end 117.801058 109.711) (width 0.2) (layer "F.Cu") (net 4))
 (segment (start 137.05 93.61) (end 136.700058 93.61) (width 0.2) (layer "F.Cu") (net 4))
 (segment (start 117.05 108.959942) (end 117.05 108.61) (width 0.2) (layer "F.Cu") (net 4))
 (segment (start 141.05 81.5325) (end 134.6275 81.5325) (width 0.2) (layer "F.Cu") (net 4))
 (segment (start 113.05 104.61) (end 112.55 104.61) (width 0.2) (layer "F.Cu") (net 4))
 (segment (start 143.5 59.945) (end 147.445 56) (width 0.2) (layer "F.Cu") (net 4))
 (segment (start 132.05 84.61) (end 131.05 84.61) (width 0.2) (layer "F.Cu") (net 4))
 (segment (start 161 56) (end 168.62 63.62) (width 0.2) (layer "F.Cu") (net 4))
 (segment (start 124.05 85.61) (end 124.05 84.61) (width 0.2) (layer "F.Cu") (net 4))
 (segment (start 124.05 84.61) (end 120.05 84.61) (width 0.2) (layer "F.Cu") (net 4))
 (segment (start 138.241 94.801) (end 137.05 93.61) (width 0.2) (layer "F.Cu") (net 4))
 (segment (start 111.949 104.009) (end 111.949 98.361058) (width 0.2) (layer "F.Cu") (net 4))
 (segment (start 162.5 96.8) (end 159.2 93.5) (width 0.2) (layer "F.Cu") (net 4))
 (segment (start 149.479 94.801) (end 138.241 94.801) (width 0.2) (layer "F.Cu") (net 4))
 (segment (start 137.05 100.61) (end 135.55 100.61) (width 0.2) (layer "F.Cu") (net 4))
 (segment (start 130.298942 85.711) (end 127.651 85.711) (width 0.2) (layer "F.Cu") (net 4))
 (segment (start 132.05 84.11) (end 132.05 84.61) (width 0.2) (layer "F.Cu") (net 4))
 (segment (start 128.05 108.11) (end 128.05 108.61) (width 0.2) (layer "F.Cu") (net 4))
 (segment (start 126.05 84.61) (end 126.05 84.959942) (width 0.2) (layer "F.Cu") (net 4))
 (segment (start 131.05 84.61) (end 131.05 84.959942) (width 0.2) (layer "F.Cu") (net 4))
 (segment (start 117.801058 109.711) (end 117.05 108.959942) (width 0.2) (layer "F.Cu") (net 4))
 (segment (start 131.05 84.959942) (end 130.298942 85.711) (width 0.2) (layer "F.Cu") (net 4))
 (segment (start 135.55 100.61) (end 128.05 108.11) (width 0.2) (layer "F.Cu") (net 4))
 (segment (start 147.445 56) (end 161 56) (width 0.2) (layer "F.Cu") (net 4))
 (segment (start 150.78 93.5) (end 149.479 94.801) (width 0.2) (layer "F.Cu") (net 4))
 (segment (start 126.05 84.959942) (end 125.298942 85.711) (width 0.2) (layer "F.Cu") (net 4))
 (segment (start 112.55 104.61) (end 111.949 104.009) (width 0.2) (layer "F.Cu") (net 4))
 (segment (start 132.05 88.959942) (end 132.05 84.61) (width 0.2) (layer "F.Cu") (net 4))
 (segment (start 127.05 84.61) (end 126.05 84.61) (width 0.2) (layer "F.Cu") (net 4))
 (segment (start 127.651 85.711) (end 127.05 85.11) (width 0.2) (layer "F.Cu") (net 4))
 (segment (start 148.67 76.4525) (end 146.13 76.4525) (width 0.2) (layer "B.Cu") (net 4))
 (segment (start 143.5 60.5) (end 143.5 59.945) (width 0.2) (layer "B.Cu") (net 4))
 (segment (start 137.945001 68.445001) (end 146 76.5) (width 0.2) (layer "B.Cu") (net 4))
 (segment (start 146.13 76.4525) (end 141.05 81.5325) (width 0.2) (layer "B.Cu") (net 4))
 (segment (start 137.945001 65.499999) (end 137.945001 68.445001) (width 0.2) (layer "B.Cu") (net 4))
 (segment (start 137.945001 65.499999) (end 143.5 59.945) (width 0.2) (layer "B.Cu") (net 4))
 (segment (start 130 65.499999) (end 137.945001 65.499999) (width 0.2) (layer "B.Cu") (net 4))
 (segment (start 161 71.24) (end 162.5 72.74) (width 0.2) (layer "F.Cu") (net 9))
 (segment (start 162.5 72.74) (end 162.5 89.2) (width 0.2) (layer "F.Cu") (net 9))
 (segment (start 162.5 89) (end 162.5 89.2) (width 0.2) (layer "B.Cu") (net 9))
 (segment (start 159.899 75.821) (end 142.22 93.5) (width 0.2) (layer "F.Cu") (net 8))
 (segment (start 159.899 69.801) (end 159.899 75.821) (width 0.2) (layer "F.Cu") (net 8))
 (segment (start 161 68.7) (end 159.899 69.801) (width 0.2) (layer "F.Cu") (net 8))
 (segment (start 146.04 59.945) (end 159.595 59.945) (width 0.2) (layer "F.Cu") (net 11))
 (segment (start 159.595 59.945) (end 161 58.54) (width 0.2) (layer "F.Cu") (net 11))
 (segment (start 159.899 57.439) (end 159.899 54.561) (width 0.2) (layer "B.Cu") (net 11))
 (segment (start 159.899 54.561) (end 161 53.46) (width 0.2) (layer "B.Cu") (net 11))
 (segment (start 146.04 59.945) (end 146.055 59.945) (width 0.2) (layer "B.Cu") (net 11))
 (segment (start 161 58.54) (end 159.899 57.439) (width 0.2) (layer "B.Cu") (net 11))
 (segment (start 161 61.08) (end 161 63.62) (width 0.2) (layer "B.Cu") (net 65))
 (segment (start 160.0635 67.599) (end 148.67 78.9925) (width 0.2) (layer "F.Cu") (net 6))
 (segment (start 168.62 68.7) (end 167.519 67.599) (width 0.2) (layer "F.Cu") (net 6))
 (segment (start 167.519 67.599) (end 160.0635 67.599) (width 0.2) (layer "F.Cu") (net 6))
 (segment (start 106.5 90.56) (end 106.5 53.5) (width 0.2) (layer "F.Cu") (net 20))
 (segment (start 106.5 53.5) (end 111.62 48.38) (width 0.2) (layer "F.Cu") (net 20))
 (segment (start 113.05 96.61) (end 112.55 96.61) (width 0.2) (layer "F.Cu") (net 20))
 (segment (start 112.55 96.61) (end 106.5 90.56) (width 0.2) (layer "F.Cu") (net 20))
 (segment (start 111.62 48.38) (end 161 48.38) (width 0.2) (layer "F.Cu") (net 20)))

